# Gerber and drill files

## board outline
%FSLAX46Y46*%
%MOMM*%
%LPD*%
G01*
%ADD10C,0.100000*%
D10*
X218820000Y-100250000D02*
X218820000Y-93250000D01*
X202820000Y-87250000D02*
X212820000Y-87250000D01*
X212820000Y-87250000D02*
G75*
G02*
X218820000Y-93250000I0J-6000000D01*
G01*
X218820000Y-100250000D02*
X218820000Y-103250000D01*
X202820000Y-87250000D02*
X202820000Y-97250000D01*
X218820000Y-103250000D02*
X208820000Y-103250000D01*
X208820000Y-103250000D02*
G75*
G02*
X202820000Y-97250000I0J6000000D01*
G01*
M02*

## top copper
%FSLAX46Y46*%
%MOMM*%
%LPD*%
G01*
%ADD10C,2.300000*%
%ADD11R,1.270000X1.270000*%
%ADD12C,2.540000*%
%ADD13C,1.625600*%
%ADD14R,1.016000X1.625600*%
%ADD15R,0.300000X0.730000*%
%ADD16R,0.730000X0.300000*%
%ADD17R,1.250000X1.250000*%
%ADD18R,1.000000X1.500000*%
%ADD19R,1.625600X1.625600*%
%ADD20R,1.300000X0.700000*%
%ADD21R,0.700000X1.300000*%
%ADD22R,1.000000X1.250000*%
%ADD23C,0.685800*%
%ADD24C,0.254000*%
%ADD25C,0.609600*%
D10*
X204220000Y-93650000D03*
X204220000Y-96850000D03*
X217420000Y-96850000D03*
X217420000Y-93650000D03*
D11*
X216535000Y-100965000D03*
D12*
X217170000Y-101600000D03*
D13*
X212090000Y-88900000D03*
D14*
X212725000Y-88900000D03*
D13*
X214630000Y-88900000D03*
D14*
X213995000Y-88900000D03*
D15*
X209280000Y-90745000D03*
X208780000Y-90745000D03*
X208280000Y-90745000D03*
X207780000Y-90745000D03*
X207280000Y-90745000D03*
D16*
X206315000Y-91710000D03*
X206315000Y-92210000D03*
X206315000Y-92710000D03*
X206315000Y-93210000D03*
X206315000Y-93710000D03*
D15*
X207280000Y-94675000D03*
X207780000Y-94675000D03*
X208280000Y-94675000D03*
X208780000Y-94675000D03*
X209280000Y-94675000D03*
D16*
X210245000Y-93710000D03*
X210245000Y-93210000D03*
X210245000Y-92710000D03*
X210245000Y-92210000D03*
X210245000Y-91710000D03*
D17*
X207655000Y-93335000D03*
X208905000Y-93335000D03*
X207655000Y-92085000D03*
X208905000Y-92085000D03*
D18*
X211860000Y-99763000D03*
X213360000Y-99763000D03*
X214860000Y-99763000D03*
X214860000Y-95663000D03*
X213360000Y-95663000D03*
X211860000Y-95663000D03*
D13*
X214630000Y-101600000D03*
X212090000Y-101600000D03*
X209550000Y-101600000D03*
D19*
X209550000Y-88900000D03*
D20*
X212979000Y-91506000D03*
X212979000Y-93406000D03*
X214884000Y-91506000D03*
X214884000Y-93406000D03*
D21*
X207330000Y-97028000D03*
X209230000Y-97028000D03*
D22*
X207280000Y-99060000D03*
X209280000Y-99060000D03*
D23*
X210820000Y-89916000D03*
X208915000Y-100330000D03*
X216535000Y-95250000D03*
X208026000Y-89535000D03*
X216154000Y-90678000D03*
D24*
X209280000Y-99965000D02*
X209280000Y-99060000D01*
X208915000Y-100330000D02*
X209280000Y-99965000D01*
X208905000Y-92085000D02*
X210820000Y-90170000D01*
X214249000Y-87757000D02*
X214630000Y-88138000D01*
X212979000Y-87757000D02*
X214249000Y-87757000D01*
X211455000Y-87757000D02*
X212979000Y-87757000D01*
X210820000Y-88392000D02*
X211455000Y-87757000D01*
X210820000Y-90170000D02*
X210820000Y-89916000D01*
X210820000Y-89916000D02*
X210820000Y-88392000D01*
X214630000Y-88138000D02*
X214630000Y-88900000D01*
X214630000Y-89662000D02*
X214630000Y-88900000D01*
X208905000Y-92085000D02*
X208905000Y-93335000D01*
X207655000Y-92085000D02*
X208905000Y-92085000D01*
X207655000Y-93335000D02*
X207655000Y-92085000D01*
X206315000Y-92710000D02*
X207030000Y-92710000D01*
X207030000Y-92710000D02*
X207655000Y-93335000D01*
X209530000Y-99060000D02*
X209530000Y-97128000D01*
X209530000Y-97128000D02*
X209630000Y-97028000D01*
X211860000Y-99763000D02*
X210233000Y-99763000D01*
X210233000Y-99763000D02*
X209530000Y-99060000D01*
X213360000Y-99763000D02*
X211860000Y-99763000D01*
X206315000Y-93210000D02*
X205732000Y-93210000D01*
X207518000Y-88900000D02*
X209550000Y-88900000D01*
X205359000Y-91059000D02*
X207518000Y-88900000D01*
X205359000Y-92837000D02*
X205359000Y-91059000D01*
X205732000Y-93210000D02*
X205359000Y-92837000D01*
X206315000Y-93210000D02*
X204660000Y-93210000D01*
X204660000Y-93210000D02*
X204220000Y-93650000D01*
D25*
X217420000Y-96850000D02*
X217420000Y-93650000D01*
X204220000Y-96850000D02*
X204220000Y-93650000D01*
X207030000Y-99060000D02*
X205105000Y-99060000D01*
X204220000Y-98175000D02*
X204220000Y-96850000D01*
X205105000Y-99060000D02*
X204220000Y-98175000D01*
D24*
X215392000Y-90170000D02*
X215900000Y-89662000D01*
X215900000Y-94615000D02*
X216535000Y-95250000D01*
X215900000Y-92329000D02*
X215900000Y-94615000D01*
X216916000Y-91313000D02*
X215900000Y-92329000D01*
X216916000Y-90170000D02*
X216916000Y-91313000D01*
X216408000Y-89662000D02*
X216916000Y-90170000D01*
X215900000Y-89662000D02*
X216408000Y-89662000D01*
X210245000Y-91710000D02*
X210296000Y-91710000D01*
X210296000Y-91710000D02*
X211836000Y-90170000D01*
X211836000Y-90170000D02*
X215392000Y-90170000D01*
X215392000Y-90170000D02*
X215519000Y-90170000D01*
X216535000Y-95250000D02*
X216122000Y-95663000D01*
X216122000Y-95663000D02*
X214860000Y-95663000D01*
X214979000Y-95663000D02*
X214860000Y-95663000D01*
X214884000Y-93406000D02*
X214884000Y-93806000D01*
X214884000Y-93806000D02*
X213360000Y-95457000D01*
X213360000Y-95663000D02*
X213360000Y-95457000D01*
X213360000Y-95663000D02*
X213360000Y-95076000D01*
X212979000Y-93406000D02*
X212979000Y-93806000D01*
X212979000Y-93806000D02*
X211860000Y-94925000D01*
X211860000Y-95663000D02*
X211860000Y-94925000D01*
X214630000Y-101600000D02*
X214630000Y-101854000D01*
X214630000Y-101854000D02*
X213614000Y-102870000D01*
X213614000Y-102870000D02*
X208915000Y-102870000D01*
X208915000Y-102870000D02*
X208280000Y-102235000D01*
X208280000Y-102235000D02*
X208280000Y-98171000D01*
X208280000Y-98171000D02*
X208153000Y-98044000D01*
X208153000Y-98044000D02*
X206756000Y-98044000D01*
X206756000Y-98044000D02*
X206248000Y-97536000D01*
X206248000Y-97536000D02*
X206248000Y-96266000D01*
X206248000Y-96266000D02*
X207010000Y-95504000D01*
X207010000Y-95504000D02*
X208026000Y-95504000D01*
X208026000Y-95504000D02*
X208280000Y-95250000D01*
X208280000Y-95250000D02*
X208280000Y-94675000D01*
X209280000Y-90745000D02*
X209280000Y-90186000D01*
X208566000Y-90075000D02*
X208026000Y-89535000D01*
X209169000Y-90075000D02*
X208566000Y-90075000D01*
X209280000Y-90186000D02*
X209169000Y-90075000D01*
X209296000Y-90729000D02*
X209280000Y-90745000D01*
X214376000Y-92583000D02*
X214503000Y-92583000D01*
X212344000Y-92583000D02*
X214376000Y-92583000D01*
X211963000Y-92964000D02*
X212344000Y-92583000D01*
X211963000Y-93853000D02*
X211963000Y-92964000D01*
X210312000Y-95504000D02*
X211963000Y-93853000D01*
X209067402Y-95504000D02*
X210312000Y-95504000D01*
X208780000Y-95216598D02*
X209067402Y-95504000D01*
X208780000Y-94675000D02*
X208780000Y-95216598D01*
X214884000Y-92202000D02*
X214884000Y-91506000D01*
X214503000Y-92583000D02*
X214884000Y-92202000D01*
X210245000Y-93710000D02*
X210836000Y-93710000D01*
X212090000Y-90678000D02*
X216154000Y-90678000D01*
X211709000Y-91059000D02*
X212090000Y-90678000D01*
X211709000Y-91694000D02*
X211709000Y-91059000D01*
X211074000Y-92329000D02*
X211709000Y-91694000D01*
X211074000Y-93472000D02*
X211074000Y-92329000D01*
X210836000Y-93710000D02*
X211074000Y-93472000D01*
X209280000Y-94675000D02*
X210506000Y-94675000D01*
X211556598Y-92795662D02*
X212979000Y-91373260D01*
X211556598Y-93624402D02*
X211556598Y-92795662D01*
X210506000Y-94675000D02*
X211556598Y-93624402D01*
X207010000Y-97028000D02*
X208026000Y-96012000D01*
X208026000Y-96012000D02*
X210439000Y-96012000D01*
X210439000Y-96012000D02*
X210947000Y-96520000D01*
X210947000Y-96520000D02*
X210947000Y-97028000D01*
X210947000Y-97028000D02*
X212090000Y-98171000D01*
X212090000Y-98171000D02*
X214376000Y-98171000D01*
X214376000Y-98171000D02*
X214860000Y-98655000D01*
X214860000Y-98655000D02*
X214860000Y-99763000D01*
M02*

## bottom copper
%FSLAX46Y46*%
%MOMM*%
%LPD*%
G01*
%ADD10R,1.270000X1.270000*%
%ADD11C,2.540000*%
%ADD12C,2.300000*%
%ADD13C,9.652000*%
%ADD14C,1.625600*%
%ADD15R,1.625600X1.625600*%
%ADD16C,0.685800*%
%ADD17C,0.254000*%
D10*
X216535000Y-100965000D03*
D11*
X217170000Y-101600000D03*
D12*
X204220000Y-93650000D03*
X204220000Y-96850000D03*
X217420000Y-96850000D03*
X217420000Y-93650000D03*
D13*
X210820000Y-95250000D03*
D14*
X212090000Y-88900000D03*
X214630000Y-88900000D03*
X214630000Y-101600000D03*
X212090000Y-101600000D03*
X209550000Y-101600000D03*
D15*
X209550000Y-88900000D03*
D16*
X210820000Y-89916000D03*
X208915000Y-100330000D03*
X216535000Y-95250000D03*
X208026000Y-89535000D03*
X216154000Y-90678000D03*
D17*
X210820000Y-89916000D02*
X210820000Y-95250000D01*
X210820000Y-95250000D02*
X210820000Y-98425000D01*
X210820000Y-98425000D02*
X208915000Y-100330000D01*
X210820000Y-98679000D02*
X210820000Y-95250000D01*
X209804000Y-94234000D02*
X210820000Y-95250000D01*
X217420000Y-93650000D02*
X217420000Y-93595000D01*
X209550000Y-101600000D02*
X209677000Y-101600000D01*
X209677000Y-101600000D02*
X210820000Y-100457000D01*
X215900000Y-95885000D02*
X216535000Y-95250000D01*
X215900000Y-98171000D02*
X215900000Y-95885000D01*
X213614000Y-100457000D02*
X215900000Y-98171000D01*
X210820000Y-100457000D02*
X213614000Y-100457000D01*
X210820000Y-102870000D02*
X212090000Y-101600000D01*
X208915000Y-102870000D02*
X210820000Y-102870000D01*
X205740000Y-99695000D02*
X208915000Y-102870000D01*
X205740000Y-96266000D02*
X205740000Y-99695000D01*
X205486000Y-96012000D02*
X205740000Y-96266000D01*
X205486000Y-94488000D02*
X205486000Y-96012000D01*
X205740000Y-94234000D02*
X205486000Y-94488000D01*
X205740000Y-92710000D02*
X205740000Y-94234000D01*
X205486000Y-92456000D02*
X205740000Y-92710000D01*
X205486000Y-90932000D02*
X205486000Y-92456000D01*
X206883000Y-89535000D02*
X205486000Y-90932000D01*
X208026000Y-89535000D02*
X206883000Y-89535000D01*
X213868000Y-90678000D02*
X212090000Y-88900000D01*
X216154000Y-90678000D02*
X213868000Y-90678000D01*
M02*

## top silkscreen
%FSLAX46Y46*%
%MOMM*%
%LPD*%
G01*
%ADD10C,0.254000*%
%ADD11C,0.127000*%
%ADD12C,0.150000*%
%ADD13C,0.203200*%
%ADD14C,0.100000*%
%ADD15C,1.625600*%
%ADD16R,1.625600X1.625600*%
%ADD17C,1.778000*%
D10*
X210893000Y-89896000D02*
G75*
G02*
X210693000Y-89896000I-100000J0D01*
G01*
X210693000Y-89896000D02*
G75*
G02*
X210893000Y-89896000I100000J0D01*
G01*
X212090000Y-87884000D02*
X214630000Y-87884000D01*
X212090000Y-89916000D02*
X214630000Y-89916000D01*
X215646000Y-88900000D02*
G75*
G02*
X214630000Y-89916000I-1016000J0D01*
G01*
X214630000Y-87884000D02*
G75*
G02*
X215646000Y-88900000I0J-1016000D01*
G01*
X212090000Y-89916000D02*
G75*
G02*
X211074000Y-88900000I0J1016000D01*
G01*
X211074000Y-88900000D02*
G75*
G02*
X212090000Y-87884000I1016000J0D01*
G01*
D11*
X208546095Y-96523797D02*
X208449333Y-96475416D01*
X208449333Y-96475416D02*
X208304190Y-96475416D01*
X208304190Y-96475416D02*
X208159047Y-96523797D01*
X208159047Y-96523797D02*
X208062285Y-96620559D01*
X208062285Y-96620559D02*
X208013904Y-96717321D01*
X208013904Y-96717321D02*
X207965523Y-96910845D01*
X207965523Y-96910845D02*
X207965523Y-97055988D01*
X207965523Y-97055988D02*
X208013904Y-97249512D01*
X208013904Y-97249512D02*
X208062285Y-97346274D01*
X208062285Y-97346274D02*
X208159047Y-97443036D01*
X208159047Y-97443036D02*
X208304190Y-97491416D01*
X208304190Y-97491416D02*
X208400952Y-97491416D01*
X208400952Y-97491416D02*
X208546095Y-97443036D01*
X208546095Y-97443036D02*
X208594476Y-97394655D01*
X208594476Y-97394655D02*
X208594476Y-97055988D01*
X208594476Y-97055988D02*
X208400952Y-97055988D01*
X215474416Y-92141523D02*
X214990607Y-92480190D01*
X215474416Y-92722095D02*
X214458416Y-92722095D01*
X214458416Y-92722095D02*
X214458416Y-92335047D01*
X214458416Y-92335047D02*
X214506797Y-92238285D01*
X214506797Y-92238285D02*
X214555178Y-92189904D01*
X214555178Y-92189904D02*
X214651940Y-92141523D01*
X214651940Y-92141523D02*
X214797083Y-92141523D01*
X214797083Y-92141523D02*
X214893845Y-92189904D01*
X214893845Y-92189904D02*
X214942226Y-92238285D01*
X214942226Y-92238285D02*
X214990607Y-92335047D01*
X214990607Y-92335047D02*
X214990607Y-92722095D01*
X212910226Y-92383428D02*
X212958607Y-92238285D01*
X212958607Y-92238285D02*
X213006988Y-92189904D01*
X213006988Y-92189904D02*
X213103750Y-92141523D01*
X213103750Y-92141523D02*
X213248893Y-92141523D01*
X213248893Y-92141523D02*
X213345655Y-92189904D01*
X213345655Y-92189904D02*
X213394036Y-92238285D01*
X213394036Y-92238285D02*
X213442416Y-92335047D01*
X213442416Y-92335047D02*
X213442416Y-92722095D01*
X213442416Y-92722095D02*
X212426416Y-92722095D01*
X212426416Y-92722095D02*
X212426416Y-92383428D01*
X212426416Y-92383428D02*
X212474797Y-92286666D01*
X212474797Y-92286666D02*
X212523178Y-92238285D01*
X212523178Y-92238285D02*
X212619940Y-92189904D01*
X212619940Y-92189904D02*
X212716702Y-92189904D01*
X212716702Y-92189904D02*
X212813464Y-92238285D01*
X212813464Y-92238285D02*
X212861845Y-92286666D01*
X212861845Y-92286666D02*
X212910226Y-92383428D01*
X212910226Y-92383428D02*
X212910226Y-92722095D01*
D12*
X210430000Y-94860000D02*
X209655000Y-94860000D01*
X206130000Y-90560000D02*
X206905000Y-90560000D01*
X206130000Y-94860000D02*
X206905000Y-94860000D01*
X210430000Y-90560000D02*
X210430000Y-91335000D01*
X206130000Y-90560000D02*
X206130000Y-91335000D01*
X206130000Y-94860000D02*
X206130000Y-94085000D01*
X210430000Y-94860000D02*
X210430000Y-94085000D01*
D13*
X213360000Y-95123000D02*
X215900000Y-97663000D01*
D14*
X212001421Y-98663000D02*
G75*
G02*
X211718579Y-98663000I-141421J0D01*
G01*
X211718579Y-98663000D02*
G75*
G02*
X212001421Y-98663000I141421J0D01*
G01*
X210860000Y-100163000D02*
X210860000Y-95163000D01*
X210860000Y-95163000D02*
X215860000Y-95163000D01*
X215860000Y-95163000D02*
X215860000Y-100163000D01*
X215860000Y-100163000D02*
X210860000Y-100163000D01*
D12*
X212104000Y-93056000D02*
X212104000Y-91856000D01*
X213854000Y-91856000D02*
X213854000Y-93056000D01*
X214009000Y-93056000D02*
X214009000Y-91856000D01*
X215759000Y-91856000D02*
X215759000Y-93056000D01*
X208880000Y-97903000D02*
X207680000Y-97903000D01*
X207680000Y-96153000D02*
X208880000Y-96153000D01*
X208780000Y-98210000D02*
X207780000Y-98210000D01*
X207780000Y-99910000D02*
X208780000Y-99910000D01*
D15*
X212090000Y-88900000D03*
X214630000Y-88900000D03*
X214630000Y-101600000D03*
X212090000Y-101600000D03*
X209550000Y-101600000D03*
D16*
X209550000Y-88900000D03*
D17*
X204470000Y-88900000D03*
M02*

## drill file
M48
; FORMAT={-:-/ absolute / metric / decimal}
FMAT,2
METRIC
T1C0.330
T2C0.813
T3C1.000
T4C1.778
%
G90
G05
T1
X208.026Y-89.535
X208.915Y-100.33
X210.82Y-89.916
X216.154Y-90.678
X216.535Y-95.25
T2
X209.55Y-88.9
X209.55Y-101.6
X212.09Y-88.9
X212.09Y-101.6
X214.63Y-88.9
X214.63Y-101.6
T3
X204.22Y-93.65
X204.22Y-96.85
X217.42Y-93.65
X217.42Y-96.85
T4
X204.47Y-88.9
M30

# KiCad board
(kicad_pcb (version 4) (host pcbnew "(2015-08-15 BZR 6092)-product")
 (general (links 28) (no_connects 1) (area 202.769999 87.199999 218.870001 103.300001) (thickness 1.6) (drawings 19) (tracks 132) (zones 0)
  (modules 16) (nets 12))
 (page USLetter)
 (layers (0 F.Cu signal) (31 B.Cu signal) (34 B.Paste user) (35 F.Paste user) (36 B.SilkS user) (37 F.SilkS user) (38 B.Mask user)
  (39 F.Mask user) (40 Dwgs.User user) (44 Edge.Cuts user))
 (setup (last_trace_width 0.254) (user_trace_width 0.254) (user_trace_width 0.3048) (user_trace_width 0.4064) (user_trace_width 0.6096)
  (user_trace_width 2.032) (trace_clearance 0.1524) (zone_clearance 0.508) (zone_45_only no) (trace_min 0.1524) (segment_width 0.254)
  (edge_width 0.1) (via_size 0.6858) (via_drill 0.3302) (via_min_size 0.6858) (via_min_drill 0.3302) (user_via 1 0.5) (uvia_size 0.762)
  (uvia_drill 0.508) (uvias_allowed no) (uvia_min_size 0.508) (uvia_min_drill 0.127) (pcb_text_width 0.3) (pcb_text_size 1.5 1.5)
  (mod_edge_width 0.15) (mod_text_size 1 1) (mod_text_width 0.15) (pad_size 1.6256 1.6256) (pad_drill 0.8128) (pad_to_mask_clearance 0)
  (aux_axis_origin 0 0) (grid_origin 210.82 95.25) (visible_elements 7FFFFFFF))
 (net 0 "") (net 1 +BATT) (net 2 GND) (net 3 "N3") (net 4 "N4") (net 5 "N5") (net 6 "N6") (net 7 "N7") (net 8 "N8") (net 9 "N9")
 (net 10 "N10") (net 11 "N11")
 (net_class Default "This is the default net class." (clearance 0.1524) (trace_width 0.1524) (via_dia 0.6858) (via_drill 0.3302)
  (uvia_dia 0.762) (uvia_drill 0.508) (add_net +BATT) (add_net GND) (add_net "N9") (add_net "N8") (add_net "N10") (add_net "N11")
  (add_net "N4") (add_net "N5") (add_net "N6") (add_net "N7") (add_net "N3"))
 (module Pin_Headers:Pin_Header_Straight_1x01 (layer B.Cu) (at 216.535 100.965 270)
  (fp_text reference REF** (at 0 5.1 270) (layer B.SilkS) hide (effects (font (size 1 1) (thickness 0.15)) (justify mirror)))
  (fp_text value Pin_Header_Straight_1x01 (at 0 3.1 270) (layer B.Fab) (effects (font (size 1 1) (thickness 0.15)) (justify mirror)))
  (pad 1 smd rect (at 0 0 270) (size 1.27 1.27) (layers B.Cu B.Paste B.Mask))
  (pad 1 smd circle (at 0.635 -0.635 270) (size 2.54 2.54) (layers B.Cu B.Paste B.Mask)))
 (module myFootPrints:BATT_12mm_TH (layer B.Cu) (at 210.82 95.25 180)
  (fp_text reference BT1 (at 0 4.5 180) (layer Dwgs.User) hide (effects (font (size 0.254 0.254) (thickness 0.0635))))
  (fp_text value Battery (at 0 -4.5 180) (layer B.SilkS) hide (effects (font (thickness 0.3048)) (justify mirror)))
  (pad 1 thru_hole circle (at 6.6 1.6 180) (size 2.3 2.3) (drill 1) (layers *.Cu *.Mask B.SilkS) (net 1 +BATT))
  (pad 1 thru_hole circle (at 6.6 -1.6 180) (size 2.3 2.3) (drill 1) (layers *.Cu *.Mask B.SilkS) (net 1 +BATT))
  (pad 1 thru_hole circle (at -6.6 -1.6 180) (size 2.3 2.3) (drill 1) (layers *.Cu *.Mask B.SilkS) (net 1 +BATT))
  (pad 1 thru_hole circle (at -6.6 1.6 180) (size 2.3 2.3) (drill 1) (layers *.Cu *.Mask B.SilkS) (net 1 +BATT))
  (pad 2 smd circle (at 0 0 180) (size 9.652 9.652) (layers B.Cu B.Paste B.Mask) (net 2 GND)))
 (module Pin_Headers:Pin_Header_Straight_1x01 (layer F.Cu) (at 216.535 100.965)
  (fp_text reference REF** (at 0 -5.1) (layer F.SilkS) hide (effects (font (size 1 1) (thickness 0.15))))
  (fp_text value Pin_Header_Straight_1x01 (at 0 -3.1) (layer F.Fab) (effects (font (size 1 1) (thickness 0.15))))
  (pad 1 smd rect (at 0 0) (size 1.27 1.27) (layers F.Cu F.Paste F.Mask))
  (pad 1 smd circle (at 0.635 0.635) (size 2.54 2.54) (layers F.Cu F.Paste F.Mask)))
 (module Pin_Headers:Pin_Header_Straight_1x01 (layer F.Cu) (at 212.09 88.9)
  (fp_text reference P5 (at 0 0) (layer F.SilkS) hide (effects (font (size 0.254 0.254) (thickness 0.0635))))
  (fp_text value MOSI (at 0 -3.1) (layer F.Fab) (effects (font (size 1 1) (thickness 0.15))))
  (pad 1 thru_hole circle (at 0 0) (size 1.6256 1.6256) (drill 0.8128) (layers *.Cu F.SilkS F.Mask) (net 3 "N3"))
  (pad 1 smd rect (at 0.635 0) (size 1.016 1.6256) (layers F.Cu F.Paste F.Mask) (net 3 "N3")))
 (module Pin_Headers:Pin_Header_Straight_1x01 (layer F.Cu) (at 214.63 88.9)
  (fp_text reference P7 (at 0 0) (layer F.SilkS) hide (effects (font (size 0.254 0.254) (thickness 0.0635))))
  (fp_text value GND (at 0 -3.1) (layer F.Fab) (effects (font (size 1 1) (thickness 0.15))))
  (pad 1 thru_hole circle (at 0 0) (size 1.6256 1.6256) (drill 0.8128) (layers *.Cu F.SilkS F.Mask) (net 2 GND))
  (pad 1 smd rect (at -0.635 0) (size 1.016 1.6256) (layers F.Cu F.Paste F.Mask) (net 2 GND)))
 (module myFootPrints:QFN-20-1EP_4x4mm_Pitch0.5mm (layer F.Cu) (at 208.28 92.71 270)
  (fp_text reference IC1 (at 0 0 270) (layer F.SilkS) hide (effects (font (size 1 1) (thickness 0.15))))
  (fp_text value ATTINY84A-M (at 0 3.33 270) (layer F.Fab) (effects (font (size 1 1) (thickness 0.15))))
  (fp_line (start 2.15 -2.15) (end 2.15 -1.375) (layer F.SilkS) (width 0.15))
  (fp_line (start -2.15 2.15) (end -2.15 1.375) (layer F.SilkS) (width 0.15))
  (fp_line (start 2.15 2.15) (end 2.15 1.375) (layer F.SilkS) (width 0.15))
  (fp_line (start -2.15 -2.15) (end -1.375 -2.15) (layer F.SilkS) (width 0.15))
  (fp_line (start -2.15 2.15) (end -1.375 2.15) (layer F.SilkS) (width 0.15))
  (fp_line (start 2.15 2.15) (end 1.375 2.15) (layer F.SilkS) (width 0.15))
  (fp_line (start 2.15 -2.15) (end 1.375 -2.15) (layer F.SilkS) (width 0.15))
  (pad 1 smd rect (at -1.965 -1 270) (size 0.73 0.3) (layers F.Cu F.Paste F.Mask) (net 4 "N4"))
  (pad 2 smd rect (at -1.965 -0.5 270) (size 0.73 0.3) (layers F.Cu F.Paste F.Mask))
  (pad 3 smd rect (at -1.965 0 270) (size 0.73 0.3) (layers F.Cu F.Paste F.Mask))
  (pad 4 smd rect (at -1.965 0.5 270) (size 0.73 0.3) (layers F.Cu F.Paste F.Mask))
  (pad 5 smd rect (at -1.965 1 270) (size 0.73 0.3) (layers F.Cu F.Paste F.Mask))
  (pad 6 smd rect (at -1 1.965) (size 0.73 0.3) (layers F.Cu F.Paste F.Mask))
  (pad 7 smd rect (at -0.5 1.965) (size 0.73 0.3) (layers F.Cu F.Paste F.Mask))
  (pad 8 smd rect (at 0 1.965) (size 0.73 0.3) (layers F.Cu F.Paste F.Mask) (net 2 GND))
  (pad 9 smd rect (at 0.5 1.965) (size 0.73 0.3) (layers F.Cu F.Paste F.Mask) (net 1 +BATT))
  (pad 10 smd rect (at 1 1.965) (size 0.73 0.3) (layers F.Cu F.Paste F.Mask))
  (pad 11 smd rect (at 1.965 1 270) (size 0.73 0.3) (layers F.Cu F.Paste F.Mask))
  (pad 12 smd rect (at 1.965 0.5 270) (size 0.73 0.3) (layers F.Cu F.Paste F.Mask))
  (pad 13 smd rect (at 1.965 0 270) (size 0.73 0.3) (layers F.Cu F.Paste F.Mask) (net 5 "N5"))
  (pad 14 smd rect (at 1.965 -0.5 270) (size 0.73 0.3) (layers F.Cu F.Paste F.Mask) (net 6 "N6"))
  (pad 15 smd rect (at 1.965 -1 270) (size 0.73 0.3) (layers F.Cu F.Paste F.Mask) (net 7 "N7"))
  (pad 16 smd rect (at 1 -1.965) (size 0.73 0.3) (layers F.Cu F.Paste F.Mask) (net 3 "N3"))
  (pad 17 smd rect (at 0.5 -1.965) (size 0.73 0.3) (layers F.Cu F.Paste F.Mask))
  (pad 18 smd rect (at 0 -1.965) (size 0.73 0.3) (layers F.Cu F.Paste F.Mask))
  (pad 19 smd rect (at -0.5 -1.965) (size 0.73 0.3) (layers F.Cu F.Paste F.Mask))
  (pad 20 smd rect (at -1 -1.965) (size 0.73 0.3) (layers F.Cu F.Paste F.Mask) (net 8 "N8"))
  (pad 8 smd rect (at 0.625 0.625 270) (size 1.25 1.25) (layers F.Cu F.Paste F.Mask) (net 2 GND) (solder_paste_margin_ratio -0.2))
  (pad 8 smd rect (at 0.625 -0.625 270) (size 1.25 1.25) (layers F.Cu F.Paste F.Mask) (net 2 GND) (solder_paste_margin_ratio -0.2))
  (pad 8 smd rect (at -0.625 0.625 270) (size 1.25 1.25) (layers F.Cu F.Paste F.Mask) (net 2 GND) (solder_paste_margin_ratio -0.2))
  (pad 8 smd rect (at -0.625 -0.625 270) (size 1.25 1.25) (layers F.Cu F.Paste F.Mask) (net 2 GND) (solder_paste_margin_ratio -0.2)))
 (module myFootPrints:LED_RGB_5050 (layer F.Cu) (at 213.36 97.663 90)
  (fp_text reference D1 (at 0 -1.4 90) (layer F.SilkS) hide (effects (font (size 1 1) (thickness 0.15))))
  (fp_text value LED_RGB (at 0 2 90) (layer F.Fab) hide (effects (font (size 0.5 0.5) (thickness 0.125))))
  (fp_line (start 2.54 0) (end 0 2.54) (layer F.SilkS) (width 0.2032))
  (fp_circle (center -1 -1.5) (end -1.1 -1.6) (layer F.SilkS) (width 0.1))
  (fp_line (start -2.5 -2.5) (end 2.5 -2.5) (layer F.SilkS) (width 0.1))
  (fp_line (start 2.5 -2.5) (end 2.5 2.5) (layer F.SilkS) (width 0.1))
  (fp_line (start 2.5 2.5) (end -2.5 2.5) (layer F.SilkS) (width 0.1))
  (fp_line (start -2.5 2.5) (end -2.5 -2.5) (layer F.SilkS) (width 0.1))
  (pad 1 smd rect (at -2.1 -1.5 180) (size 1 1.5) (layers F.Cu F.Paste F.Mask) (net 2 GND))
  (pad 2 smd rect (at -2.1 0 180) (size 1 1.5) (layers F.Cu F.Paste F.Mask) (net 2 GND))
  (pad 3 smd rect (at -2.1 1.5 180) (size 1 1.5) (layers F.Cu F.Paste F.Mask) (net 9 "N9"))
  (pad 4 smd rect (at 2 1.5 180) (size 1 1.5) (layers F.Cu F.Paste F.Mask) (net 8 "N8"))
  (pad 5 smd rect (at 2 0 180) (size 1 1.5) (layers F.Cu F.Paste F.Mask) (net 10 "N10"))
  (pad 6 smd rect (at 2 -1.5 180) (size 1 1.5) (layers F.Cu F.Paste F.Mask) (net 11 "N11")))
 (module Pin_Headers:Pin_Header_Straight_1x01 (layer F.Cu) (at 214.63 101.6)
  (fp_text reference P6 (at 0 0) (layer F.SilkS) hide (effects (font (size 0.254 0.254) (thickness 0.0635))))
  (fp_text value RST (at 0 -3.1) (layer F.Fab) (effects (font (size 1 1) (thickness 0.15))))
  (pad 1 thru_hole circle (at 0 0) (size 1.6256 1.6256) (drill 0.8128) (layers *.Cu F.SilkS F.Mask) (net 5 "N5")))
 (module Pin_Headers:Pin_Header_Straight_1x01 (layer F.Cu) (at 212.09 101.6)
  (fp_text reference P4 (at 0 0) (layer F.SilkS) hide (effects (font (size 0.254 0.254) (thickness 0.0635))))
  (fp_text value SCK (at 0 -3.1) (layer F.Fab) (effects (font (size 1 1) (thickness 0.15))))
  (pad 1 thru_hole circle (at 0 0) (size 1.6256 1.6256) (drill 0.8128) (layers *.Cu F.SilkS F.Mask) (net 4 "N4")))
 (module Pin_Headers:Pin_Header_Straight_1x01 (layer F.Cu) (at 209.55 101.6)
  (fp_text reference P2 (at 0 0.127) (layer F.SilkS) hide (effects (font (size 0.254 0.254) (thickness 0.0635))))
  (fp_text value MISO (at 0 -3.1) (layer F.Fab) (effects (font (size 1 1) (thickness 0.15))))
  (pad 1 thru_hole circle (at 0 0) (size 1.6256 1.6256) (drill 0.8128) (layers *.Cu F.SilkS F.Mask) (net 8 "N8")))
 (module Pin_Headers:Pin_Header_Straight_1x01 (layer F.Cu) (at 209.55 88.9)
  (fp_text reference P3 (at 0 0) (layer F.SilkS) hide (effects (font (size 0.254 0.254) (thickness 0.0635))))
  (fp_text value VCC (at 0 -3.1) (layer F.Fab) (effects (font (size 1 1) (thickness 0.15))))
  (pad 1 thru_hole rect (at 0 0) (size 1.6256 1.6256) (drill 0.8128) (layers *.Cu F.SilkS F.Mask) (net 1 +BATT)))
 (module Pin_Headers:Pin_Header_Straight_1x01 (layer F.Cu) (at 204.47 88.9)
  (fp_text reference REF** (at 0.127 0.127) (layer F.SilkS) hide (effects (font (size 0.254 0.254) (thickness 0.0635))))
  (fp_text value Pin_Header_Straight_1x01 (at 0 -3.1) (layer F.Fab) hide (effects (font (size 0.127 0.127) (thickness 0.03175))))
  (pad "" np_thru_hole circle (at 0 0) (size 1.778 1.778) (drill 1.778) (layers *.Cu *.Mask F.SilkS)))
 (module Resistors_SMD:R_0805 (layer F.Cu) (at 212.979 92.456 270)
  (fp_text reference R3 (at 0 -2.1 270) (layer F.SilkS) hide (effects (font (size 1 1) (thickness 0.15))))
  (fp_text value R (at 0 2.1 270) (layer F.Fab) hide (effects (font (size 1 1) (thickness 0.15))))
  (fp_line (start 0.6 0.875) (end -0.6 0.875) (layer F.SilkS) (width 0.15))
  (fp_line (start -0.6 -0.875) (end 0.6 -0.875) (layer F.SilkS) (width 0.15))
  (pad 1 smd rect (at -0.95 0 270) (size 0.7 1.3) (layers F.Cu F.Paste F.Mask) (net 7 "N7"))
  (pad 2 smd rect (at 0.95 0 270) (size 0.7 1.3) (layers F.Cu F.Paste F.Mask) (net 11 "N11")))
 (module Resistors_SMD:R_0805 (layer F.Cu) (at 214.884 92.456 270)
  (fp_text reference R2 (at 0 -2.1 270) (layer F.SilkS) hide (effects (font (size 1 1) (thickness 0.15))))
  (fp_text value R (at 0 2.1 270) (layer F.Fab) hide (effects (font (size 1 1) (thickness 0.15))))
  (fp_line (start 0.6 0.875) (end -0.6 0.875) (layer F.SilkS) (width 0.15))
  (fp_line (start -0.6 -0.875) (end 0.6 -0.875) (layer F.SilkS) (width 0.15))
  (pad 1 smd rect (at -0.95 0 270) (size 0.7 1.3) (layers F.Cu F.Paste F.Mask) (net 6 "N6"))
  (pad 2 smd rect (at 0.95 0 270) (size 0.7 1.3) (layers F.Cu F.Paste F.Mask) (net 10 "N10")))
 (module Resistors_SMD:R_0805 (layer F.Cu) (at 208.28 97.028)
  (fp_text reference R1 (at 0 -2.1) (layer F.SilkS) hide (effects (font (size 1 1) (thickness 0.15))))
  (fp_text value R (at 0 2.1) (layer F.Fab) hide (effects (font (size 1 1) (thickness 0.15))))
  (fp_line (start 0.6 0.875) (end -0.6 0.875) (layer F.SilkS) (width 0.15))
  (fp_line (start -0.6 -0.875) (end 0.6 -0.875) (layer F.SilkS) (width 0.15))
  (pad 1 smd rect (at -0.95 0) (size 0.7 1.3) (layers F.Cu F.Paste F.Mask) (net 9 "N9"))
  (pad 2 smd rect (at 0.95 0) (size 0.7 1.3) (layers F.Cu F.Paste F.Mask) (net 2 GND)))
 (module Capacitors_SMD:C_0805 (layer F.Cu) (at 208.28 99.06)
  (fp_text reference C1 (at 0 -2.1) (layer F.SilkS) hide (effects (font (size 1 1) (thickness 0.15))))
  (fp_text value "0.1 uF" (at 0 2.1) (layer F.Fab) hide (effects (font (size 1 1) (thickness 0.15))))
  (fp_line (start 0.5 -0.85) (end -0.5 -0.85) (layer F.SilkS) (width 0.15))
  (fp_line (start -0.5 0.85) (end 0.5 0.85) (layer F.SilkS) (width 0.15))
  (pad 1 smd rect (at -1 0) (size 1 1.25) (layers F.Cu F.Paste F.Mask) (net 1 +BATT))
  (pad 2 smd rect (at 1 0) (size 1 1.25) (layers F.Cu F.Paste F.Mask) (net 2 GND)))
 (gr_line (start 218.82 100.25) (end 218.82 93.25) (angle 90) (layer Edge.Cuts) (width 0.1))
 (gr_line (start 202.82 87.25) (end 212.82 87.25) (angle 90) (layer Edge.Cuts) (width 0.1))
 (gr_arc (start 212.82 93.25) (end 212.82 87.25) (angle 90) (layer Edge.Cuts) (width 0.1))
 (gr_line (start 218.82 100.25) (end 218.82 103.25) (angle 90) (layer Edge.Cuts) (width 0.1))
 (gr_line (start 202.82 87.25) (end 202.82 97.25) (angle 90) (layer Edge.Cuts) (width 0.1))
 (gr_line (start 218.82 103.25) (end 208.82 103.25) (angle 90) (layer Edge.Cuts) (width 0.1))
 (gr_arc (start 208.82 97.25) (end 208.82 103.25) (angle 90) (layer Edge.Cuts) (width 0.1))
 (gr_circle (center 210.793 89.896) (end 210.893 89.896) (layer F.SilkS) (width 0.254))
 (gr_line (start 212.09 87.884) (end 214.63 87.884) (angle 90) (layer F.SilkS) (width 0.254))
 (gr_line (start 212.09 89.916) (end 214.63 89.916) (angle 90) (layer F.SilkS) (width 0.254))
 (gr_arc (start 214.63 88.9) (end 215.646 88.9) (angle 90) (layer F.SilkS) (width 0.254))
 (gr_arc (start 214.63 88.9) (end 214.63 87.884) (angle 90) (layer F.SilkS) (width 0.254))
 (gr_arc (start 212.09 88.9) (end 212.09 89.916) (angle 90) (layer F.SilkS) (width 0.254))
 (gr_arc (start 212.09 88.9) (end 211.074 88.9) (angle 90) (layer F.SilkS) (width 0.254))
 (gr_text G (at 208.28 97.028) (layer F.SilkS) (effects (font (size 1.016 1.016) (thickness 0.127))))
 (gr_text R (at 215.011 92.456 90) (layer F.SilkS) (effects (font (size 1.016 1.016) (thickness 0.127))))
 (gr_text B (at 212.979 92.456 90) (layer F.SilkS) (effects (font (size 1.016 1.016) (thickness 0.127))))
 (via (at 210.82 89.916) (size 0.6858) (drill 0.3302) (layers F.Cu B.Cu) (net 2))
 (segment (start 210.82 89.916) (end 210.82 95.25) (width 0.254) (layer B.Cu) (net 2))
 (segment (start 210.82 95.25) (end 210.82 98.425) (width 0.254) (layer B.Cu) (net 2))
 (segment (start 210.82 98.425) (end 208.915 100.33) (width 0.254) (layer B.Cu) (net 2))
 (segment (start 209.28 99.965) (end 209.28 99.06) (width 0.254) (layer F.Cu) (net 2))
 (segment (start 208.915 100.33) (end 209.28 99.965) (width 0.254) (layer F.Cu) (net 2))
 (via (at 208.915 100.33) (size 0.6858) (drill 0.3302) (layers F.Cu B.Cu) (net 2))
 (segment (start 208.905 92.085) (end 210.82 90.17) (width 0.254) (layer F.Cu) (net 2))
 (segment (start 214.249 87.757) (end 214.63 88.138) (width 0.254) (layer F.Cu) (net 2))
 (segment (start 212.979 87.757) (end 214.249 87.757) (width 0.254) (layer F.Cu) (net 2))
 (segment (start 211.455 87.757) (end 212.979 87.757) (width 0.254) (layer F.Cu) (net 2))
 (segment (start 210.82 88.392) (end 211.455 87.757) (width 0.254) (layer F.Cu) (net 2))
 (segment (start 210.82 90.17) (end 210.82 89.916) (width 0.254) (layer F.Cu) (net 2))
 (segment (start 210.82 89.916) (end 210.82 88.392) (width 0.254) (layer F.Cu) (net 2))
 (segment (start 214.63 88.138) (end 214.63 88.9) (width 0.254) (layer F.Cu) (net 2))
 (segment (start 214.63 89.662) (end 214.63 88.9) (width 0.254) (layer F.Cu) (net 2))
 (segment (start 208.905 92.085) (end 208.905 93.335) (width 0.254) (layer F.Cu) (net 2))
 (segment (start 207.655 92.085) (end 208.905 92.085) (width 0.254) (layer F.Cu) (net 2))
 (segment (start 207.655 93.335) (end 207.655 92.085) (width 0.254) (layer F.Cu) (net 2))
 (segment (start 206.315 92.71) (end 207.03 92.71) (width 0.254) (layer F.Cu) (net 2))
 (segment (start 207.03 92.71) (end 207.655 93.335) (width 0.254) (layer F.Cu) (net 2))
 (segment (start 210.82 98.679) (end 210.82 95.25) (width 0.254) (layer B.Cu) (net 2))
 (segment (start 209.804 94.234) (end 210.82 95.25) (width 0.254) (layer B.Cu) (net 2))
 (segment (start 209.53 99.06) (end 209.53 97.128) (width 0.254) (layer F.Cu) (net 2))
 (segment (start 209.53 97.128) (end 209.63 97.028) (width 0.254) (layer F.Cu) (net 2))
 (segment (start 211.86 99.763) (end 210.233 99.763) (width 0.254) (layer F.Cu) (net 2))
 (segment (start 210.233 99.763) (end 209.53 99.06) (width 0.254) (layer F.Cu) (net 2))
 (segment (start 213.36 99.763) (end 211.86 99.763) (width 0.254) (layer F.Cu) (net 2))
 (segment (start 206.315 93.21) (end 205.732 93.21) (width 0.254) (layer F.Cu) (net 1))
 (segment (start 207.518 88.9) (end 209.55 88.9) (width 0.254) (layer F.Cu) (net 1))
 (segment (start 205.359 91.059) (end 207.518 88.9) (width 0.254) (layer F.Cu) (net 1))
 (segment (start 205.359 92.837) (end 205.359 91.059) (width 0.254) (layer F.Cu) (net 1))
 (segment (start 205.732 93.21) (end 205.359 92.837) (width 0.254) (layer F.Cu) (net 1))
 (segment (start 217.42 93.65) (end 217.42 93.595) (width 0.254) (layer B.Cu) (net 1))
 (segment (start 206.315 93.21) (end 204.66 93.21) (width 0.254) (layer F.Cu) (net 1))
 (segment (start 204.66 93.21) (end 204.22 93.65) (width 0.254) (layer F.Cu) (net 1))
 (segment (start 217.42 96.85) (end 217.42 93.65) (width 0.6096) (layer F.Cu) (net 1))
 (segment (start 204.22 96.85) (end 204.22 93.65) (width 0.6096) (layer F.Cu) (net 1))
 (segment (start 207.03 99.06) (end 205.105 99.06) (width 0.6096) (layer F.Cu) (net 1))
 (segment (start 204.22 98.175) (end 204.22 96.85) (width 0.6096) (layer F.Cu) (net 1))
 (segment (start 205.105 99.06) (end 204.22 98.175) (width 0.6096) (layer F.Cu) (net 1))
 (segment (start 215.392 90.17) (end 215.9 89.662) (width 0.254) (layer F.Cu) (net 8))
 (segment (start 215.9 94.615) (end 216.535 95.25) (width 0.254) (layer F.Cu) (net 8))
 (segment (start 215.9 92.329) (end 215.9 94.615) (width 0.254) (layer F.Cu) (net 8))
 (segment (start 216.916 91.313) (end 215.9 92.329) (width 0.254) (layer F.Cu) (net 8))
 (segment (start 216.916 90.17) (end 216.916 91.313) (width 0.254) (layer F.Cu) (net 8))
 (segment (start 216.408 89.662) (end 216.916 90.17) (width 0.254) (layer F.Cu) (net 8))
 (segment (start 215.9 89.662) (end 216.408 89.662) (width 0.254) (layer F.Cu) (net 8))
 (segment (start 210.245 91.71) (end 210.296 91.71) (width 0.254) (layer F.Cu) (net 8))
 (segment (start 210.296 91.71) (end 211.836 90.17) (width 0.254) (layer F.Cu) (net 8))
 (segment (start 211.836 90.17) (end 215.392 90.17) (width 0.254) (layer F.Cu) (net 8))
 (segment (start 215.392 90.17) (end 215.519 90.17) (width 0.254) (layer F.Cu) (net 8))
 (segment (start 209.55 101.6) (end 209.677 101.6) (width 0.254) (layer B.Cu) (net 8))
 (segment (start 209.677 101.6) (end 210.82 100.457) (width 0.254) (layer B.Cu) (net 8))
 (via (at 216.535 95.25) (size 0.6858) (drill 0.3302) (layers F.Cu B.Cu) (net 8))
 (segment (start 215.9 95.885) (end 216.535 95.25) (width 0.254) (layer B.Cu) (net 8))
 (segment (start 215.9 98.171) (end 215.9 95.885) (width 0.254) (layer B.Cu) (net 8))
 (segment (start 213.614 100.457) (end 215.9 98.171) (width 0.254) (layer B.Cu) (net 8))
 (segment (start 210.82 100.457) (end 213.614 100.457) (width 0.254) (layer B.Cu) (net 8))
 (segment (start 216.535 95.25) (end 216.122 95.663) (width 0.254) (layer F.Cu) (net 8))
 (segment (start 216.122 95.663) (end 214.86 95.663) (width 0.254) (layer F.Cu) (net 8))
 (segment (start 214.979 95.663) (end 214.86 95.663) (width 0.254) (layer F.Cu) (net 8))
 (segment (start 214.884 93.406) (end 214.884 93.806) (width 0.254) (layer F.Cu) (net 10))
 (segment (start 214.884 93.806) (end 213.36 95.457) (width 0.254) (layer F.Cu) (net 10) (status 20))
 (segment (start 213.36 95.663) (end 213.36 95.457) (width 0.254) (layer F.Cu) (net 10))
 (segment (start 213.36 95.663) (end 213.36 95.076) (width 0.254) (layer F.Cu) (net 10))
 (segment (start 212.979 93.406) (end 212.979 93.806) (width 0.254) (layer F.Cu) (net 11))
 (segment (start 212.979 93.806) (end 211.86 94.925) (width 0.254) (layer F.Cu) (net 11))
 (segment (start 211.86 95.663) (end 211.86 94.925) (width 0.254) (layer F.Cu) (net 11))
 (segment (start 214.63 101.6) (end 214.63 101.854) (width 0.254) (layer F.Cu) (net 5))
 (segment (start 214.63 101.854) (end 213.614 102.87) (width 0.254) (layer F.Cu) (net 5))
 (segment (start 213.614 102.87) (end 208.915 102.87) (width 0.254) (layer F.Cu) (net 5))
 (segment (start 208.915 102.87) (end 208.28 102.235) (width 0.254) (layer F.Cu) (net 5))
 (segment (start 208.28 102.235) (end 208.28 98.171) (width 0.254) (layer F.Cu) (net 5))
 (segment (start 208.28 98.171) (end 208.153 98.044) (width 0.254) (layer F.Cu) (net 5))
 (segment (start 208.153 98.044) (end 206.756 98.044) (width 0.254) (layer F.Cu) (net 5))
 (segment (start 206.756 98.044) (end 206.248 97.536) (width 0.254) (layer F.Cu) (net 5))
 (segment (start 206.248 97.536) (end 206.248 96.266) (width 0.254) (layer F.Cu) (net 5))
 (segment (start 206.248 96.266) (end 207.01 95.504) (width 0.254) (layer F.Cu) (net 5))
 (segment (start 207.01 95.504) (end 208.026 95.504) (width 0.254) (layer F.Cu) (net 5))
 (segment (start 208.026 95.504) (end 208.28 95.25) (width 0.254) (layer F.Cu) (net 5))
 (segment (start 208.28 95.25) (end 208.28 94.675) (width 0.254) (layer F.Cu) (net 5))
 (segment (start 209.28 90.745) (end 209.28 90.186) (width 0.254) (layer F.Cu) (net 4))
 (segment (start 210.82 102.87) (end 212.09 101.6) (width 0.254) (layer B.Cu) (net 4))
 (segment (start 208.915 102.87) (end 210.82 102.87) (width 0.254) (layer B.Cu) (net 4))
 (segment (start 205.74 99.695) (end 208.915 102.87) (width 0.254) (layer B.Cu) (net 4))
 (segment (start 205.74 96.266) (end 205.74 99.695) (width 0.254) (layer B.Cu) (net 4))
 (segment (start 205.486 96.012) (end 205.74 96.266) (width 0.254) (layer B.Cu) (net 4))
 (segment (start 205.486 94.488) (end 205.486 96.012) (width 0.254) (layer B.Cu) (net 4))
 (segment (start 205.74 94.234) (end 205.486 94.488) (width 0.254) (layer B.Cu) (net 4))
 (segment (start 205.74 92.71) (end 205.74 94.234) (width 0.254) (layer B.Cu) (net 4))
 (segment (start 205.486 92.456) (end 205.74 92.71) (width 0.254) (layer B.Cu) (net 4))
 (segment (start 205.486 90.932) (end 205.486 92.456) (width 0.254) (layer B.Cu) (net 4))
 (segment (start 206.883 89.535) (end 205.486 90.932) (width 0.254) (layer B.Cu) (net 4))
 (segment (start 208.026 89.535) (end 206.883 89.535) (width 0.254) (layer B.Cu) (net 4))
 (via (at 208.026 89.535) (size 0.6858) (drill 0.3302) (layers F.Cu B.Cu) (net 4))
 (segment (start 208.566 90.075) (end 208.026 89.535) (width 0.254) (layer F.Cu) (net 4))
 (segment (start 209.169 90.075) (end 208.566 90.075) (width 0.254) (layer F.Cu) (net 4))
 (segment (start 209.28 90.186) (end 209.169 90.075) (width 0.254) (layer F.Cu) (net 4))
 (segment (start 209.296 90.729) (end 209.28 90.745) (width 0.254) (layer F.Cu) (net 4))
 (segment (start 214.376 92.583) (end 214.503 92.583) (width 0.254) (layer F.Cu) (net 6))
 (segment (start 212.344 92.583) (end 214.376 92.583) (width 0.254) (layer F.Cu) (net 6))
 (segment (start 211.963 92.964) (end 212.344 92.583) (width 0.254) (layer F.Cu) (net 6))
 (segment (start 211.963 93.853) (end 211.963 92.964) (width 0.254) (layer F.Cu) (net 6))
 (segment (start 210.312 95.504) (end 211.963 93.853) (width 0.254) (layer F.Cu) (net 6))
 (segment (start 209.067402 95.504) (end 210.312 95.504) (width 0.254) (layer F.Cu) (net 6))
 (segment (start 208.78 95.216598) (end 209.067402 95.504) (width 0.254) (layer F.Cu) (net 6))
 (segment (start 208.78 94.675) (end 208.78 95.216598) (width 0.254) (layer F.Cu) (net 6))
 (segment (start 214.884 92.202) (end 214.884 91.506) (width 0.254) (layer F.Cu) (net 6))
 (segment (start 214.503 92.583) (end 214.884 92.202) (width 0.254) (layer F.Cu) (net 6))
 (segment (start 210.245 93.71) (end 210.836 93.71) (width 0.254) (layer F.Cu) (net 3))
 (segment (start 213.868 90.678) (end 212.09 88.9) (width 0.254) (layer B.Cu) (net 3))
 (segment (start 216.154 90.678) (end 213.868 90.678) (width 0.254) (layer B.Cu) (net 3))
 (via (at 216.154 90.678) (size 0.6858) (drill 0.3302) (layers F.Cu B.Cu) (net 3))
 (segment (start 212.09 90.678) (end 216.154 90.678) (width 0.254) (layer F.Cu) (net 3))
 (segment (start 211.709 91.059) (end 212.09 90.678) (width 0.254) (layer F.Cu) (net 3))
 (segment (start 211.709 91.694) (end 211.709 91.059) (width 0.254) (layer F.Cu) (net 3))
 (segment (start 211.074 92.329) (end 211.709 91.694) (width 0.254) (layer F.Cu) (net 3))
 (segment (start 211.074 93.472) (end 211.074 92.329) (width 0.254) (layer F.Cu) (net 3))
 (segment (start 210.836 93.71) (end 211.074 93.472) (width 0.254) (layer F.Cu) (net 3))
 (segment (start 209.28 94.675) (end 210.506 94.675) (width 0.254) (layer F.Cu) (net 7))
 (segment (start 211.556598 92.795662) (end 212.979 91.37326) (width 0.254) (layer F.Cu) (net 7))
 (segment (start 211.556598 93.624402) (end 211.556598 92.795662) (width 0.254) (layer F.Cu) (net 7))
 (segment (start 210.506 94.675) (end 211.556598 93.624402) (width 0.254) (layer F.Cu) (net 7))
 (segment (start 207.01 97.028) (end 208.026 96.012) (width 0.254) (layer F.Cu) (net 9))
 (segment (start 208.026 96.012) (end 210.439 96.012) (width 0.254) (layer F.Cu) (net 9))
 (segment (start 210.439 96.012) (end 210.947 96.52) (width 0.254) (layer F.Cu) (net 9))
 (segment (start 210.947 96.52) (end 210.947 97.028) (width 0.254) (layer F.Cu) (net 9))
 (segment (start 210.947 97.028) (end 212.09 98.171) (width 0.254) (layer F.Cu) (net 9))
 (segment (start 212.09 98.171) (end 214.376 98.171) (width 0.254) (layer F.Cu) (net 9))
 (segment (start 214.376 98.171) (end 214.86 98.655) (width 0.254) (layer F.Cu) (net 9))
 (segment (start 214.86 98.655) (end 214.86 99.763) (width 0.254) (layer F.Cu) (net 9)))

